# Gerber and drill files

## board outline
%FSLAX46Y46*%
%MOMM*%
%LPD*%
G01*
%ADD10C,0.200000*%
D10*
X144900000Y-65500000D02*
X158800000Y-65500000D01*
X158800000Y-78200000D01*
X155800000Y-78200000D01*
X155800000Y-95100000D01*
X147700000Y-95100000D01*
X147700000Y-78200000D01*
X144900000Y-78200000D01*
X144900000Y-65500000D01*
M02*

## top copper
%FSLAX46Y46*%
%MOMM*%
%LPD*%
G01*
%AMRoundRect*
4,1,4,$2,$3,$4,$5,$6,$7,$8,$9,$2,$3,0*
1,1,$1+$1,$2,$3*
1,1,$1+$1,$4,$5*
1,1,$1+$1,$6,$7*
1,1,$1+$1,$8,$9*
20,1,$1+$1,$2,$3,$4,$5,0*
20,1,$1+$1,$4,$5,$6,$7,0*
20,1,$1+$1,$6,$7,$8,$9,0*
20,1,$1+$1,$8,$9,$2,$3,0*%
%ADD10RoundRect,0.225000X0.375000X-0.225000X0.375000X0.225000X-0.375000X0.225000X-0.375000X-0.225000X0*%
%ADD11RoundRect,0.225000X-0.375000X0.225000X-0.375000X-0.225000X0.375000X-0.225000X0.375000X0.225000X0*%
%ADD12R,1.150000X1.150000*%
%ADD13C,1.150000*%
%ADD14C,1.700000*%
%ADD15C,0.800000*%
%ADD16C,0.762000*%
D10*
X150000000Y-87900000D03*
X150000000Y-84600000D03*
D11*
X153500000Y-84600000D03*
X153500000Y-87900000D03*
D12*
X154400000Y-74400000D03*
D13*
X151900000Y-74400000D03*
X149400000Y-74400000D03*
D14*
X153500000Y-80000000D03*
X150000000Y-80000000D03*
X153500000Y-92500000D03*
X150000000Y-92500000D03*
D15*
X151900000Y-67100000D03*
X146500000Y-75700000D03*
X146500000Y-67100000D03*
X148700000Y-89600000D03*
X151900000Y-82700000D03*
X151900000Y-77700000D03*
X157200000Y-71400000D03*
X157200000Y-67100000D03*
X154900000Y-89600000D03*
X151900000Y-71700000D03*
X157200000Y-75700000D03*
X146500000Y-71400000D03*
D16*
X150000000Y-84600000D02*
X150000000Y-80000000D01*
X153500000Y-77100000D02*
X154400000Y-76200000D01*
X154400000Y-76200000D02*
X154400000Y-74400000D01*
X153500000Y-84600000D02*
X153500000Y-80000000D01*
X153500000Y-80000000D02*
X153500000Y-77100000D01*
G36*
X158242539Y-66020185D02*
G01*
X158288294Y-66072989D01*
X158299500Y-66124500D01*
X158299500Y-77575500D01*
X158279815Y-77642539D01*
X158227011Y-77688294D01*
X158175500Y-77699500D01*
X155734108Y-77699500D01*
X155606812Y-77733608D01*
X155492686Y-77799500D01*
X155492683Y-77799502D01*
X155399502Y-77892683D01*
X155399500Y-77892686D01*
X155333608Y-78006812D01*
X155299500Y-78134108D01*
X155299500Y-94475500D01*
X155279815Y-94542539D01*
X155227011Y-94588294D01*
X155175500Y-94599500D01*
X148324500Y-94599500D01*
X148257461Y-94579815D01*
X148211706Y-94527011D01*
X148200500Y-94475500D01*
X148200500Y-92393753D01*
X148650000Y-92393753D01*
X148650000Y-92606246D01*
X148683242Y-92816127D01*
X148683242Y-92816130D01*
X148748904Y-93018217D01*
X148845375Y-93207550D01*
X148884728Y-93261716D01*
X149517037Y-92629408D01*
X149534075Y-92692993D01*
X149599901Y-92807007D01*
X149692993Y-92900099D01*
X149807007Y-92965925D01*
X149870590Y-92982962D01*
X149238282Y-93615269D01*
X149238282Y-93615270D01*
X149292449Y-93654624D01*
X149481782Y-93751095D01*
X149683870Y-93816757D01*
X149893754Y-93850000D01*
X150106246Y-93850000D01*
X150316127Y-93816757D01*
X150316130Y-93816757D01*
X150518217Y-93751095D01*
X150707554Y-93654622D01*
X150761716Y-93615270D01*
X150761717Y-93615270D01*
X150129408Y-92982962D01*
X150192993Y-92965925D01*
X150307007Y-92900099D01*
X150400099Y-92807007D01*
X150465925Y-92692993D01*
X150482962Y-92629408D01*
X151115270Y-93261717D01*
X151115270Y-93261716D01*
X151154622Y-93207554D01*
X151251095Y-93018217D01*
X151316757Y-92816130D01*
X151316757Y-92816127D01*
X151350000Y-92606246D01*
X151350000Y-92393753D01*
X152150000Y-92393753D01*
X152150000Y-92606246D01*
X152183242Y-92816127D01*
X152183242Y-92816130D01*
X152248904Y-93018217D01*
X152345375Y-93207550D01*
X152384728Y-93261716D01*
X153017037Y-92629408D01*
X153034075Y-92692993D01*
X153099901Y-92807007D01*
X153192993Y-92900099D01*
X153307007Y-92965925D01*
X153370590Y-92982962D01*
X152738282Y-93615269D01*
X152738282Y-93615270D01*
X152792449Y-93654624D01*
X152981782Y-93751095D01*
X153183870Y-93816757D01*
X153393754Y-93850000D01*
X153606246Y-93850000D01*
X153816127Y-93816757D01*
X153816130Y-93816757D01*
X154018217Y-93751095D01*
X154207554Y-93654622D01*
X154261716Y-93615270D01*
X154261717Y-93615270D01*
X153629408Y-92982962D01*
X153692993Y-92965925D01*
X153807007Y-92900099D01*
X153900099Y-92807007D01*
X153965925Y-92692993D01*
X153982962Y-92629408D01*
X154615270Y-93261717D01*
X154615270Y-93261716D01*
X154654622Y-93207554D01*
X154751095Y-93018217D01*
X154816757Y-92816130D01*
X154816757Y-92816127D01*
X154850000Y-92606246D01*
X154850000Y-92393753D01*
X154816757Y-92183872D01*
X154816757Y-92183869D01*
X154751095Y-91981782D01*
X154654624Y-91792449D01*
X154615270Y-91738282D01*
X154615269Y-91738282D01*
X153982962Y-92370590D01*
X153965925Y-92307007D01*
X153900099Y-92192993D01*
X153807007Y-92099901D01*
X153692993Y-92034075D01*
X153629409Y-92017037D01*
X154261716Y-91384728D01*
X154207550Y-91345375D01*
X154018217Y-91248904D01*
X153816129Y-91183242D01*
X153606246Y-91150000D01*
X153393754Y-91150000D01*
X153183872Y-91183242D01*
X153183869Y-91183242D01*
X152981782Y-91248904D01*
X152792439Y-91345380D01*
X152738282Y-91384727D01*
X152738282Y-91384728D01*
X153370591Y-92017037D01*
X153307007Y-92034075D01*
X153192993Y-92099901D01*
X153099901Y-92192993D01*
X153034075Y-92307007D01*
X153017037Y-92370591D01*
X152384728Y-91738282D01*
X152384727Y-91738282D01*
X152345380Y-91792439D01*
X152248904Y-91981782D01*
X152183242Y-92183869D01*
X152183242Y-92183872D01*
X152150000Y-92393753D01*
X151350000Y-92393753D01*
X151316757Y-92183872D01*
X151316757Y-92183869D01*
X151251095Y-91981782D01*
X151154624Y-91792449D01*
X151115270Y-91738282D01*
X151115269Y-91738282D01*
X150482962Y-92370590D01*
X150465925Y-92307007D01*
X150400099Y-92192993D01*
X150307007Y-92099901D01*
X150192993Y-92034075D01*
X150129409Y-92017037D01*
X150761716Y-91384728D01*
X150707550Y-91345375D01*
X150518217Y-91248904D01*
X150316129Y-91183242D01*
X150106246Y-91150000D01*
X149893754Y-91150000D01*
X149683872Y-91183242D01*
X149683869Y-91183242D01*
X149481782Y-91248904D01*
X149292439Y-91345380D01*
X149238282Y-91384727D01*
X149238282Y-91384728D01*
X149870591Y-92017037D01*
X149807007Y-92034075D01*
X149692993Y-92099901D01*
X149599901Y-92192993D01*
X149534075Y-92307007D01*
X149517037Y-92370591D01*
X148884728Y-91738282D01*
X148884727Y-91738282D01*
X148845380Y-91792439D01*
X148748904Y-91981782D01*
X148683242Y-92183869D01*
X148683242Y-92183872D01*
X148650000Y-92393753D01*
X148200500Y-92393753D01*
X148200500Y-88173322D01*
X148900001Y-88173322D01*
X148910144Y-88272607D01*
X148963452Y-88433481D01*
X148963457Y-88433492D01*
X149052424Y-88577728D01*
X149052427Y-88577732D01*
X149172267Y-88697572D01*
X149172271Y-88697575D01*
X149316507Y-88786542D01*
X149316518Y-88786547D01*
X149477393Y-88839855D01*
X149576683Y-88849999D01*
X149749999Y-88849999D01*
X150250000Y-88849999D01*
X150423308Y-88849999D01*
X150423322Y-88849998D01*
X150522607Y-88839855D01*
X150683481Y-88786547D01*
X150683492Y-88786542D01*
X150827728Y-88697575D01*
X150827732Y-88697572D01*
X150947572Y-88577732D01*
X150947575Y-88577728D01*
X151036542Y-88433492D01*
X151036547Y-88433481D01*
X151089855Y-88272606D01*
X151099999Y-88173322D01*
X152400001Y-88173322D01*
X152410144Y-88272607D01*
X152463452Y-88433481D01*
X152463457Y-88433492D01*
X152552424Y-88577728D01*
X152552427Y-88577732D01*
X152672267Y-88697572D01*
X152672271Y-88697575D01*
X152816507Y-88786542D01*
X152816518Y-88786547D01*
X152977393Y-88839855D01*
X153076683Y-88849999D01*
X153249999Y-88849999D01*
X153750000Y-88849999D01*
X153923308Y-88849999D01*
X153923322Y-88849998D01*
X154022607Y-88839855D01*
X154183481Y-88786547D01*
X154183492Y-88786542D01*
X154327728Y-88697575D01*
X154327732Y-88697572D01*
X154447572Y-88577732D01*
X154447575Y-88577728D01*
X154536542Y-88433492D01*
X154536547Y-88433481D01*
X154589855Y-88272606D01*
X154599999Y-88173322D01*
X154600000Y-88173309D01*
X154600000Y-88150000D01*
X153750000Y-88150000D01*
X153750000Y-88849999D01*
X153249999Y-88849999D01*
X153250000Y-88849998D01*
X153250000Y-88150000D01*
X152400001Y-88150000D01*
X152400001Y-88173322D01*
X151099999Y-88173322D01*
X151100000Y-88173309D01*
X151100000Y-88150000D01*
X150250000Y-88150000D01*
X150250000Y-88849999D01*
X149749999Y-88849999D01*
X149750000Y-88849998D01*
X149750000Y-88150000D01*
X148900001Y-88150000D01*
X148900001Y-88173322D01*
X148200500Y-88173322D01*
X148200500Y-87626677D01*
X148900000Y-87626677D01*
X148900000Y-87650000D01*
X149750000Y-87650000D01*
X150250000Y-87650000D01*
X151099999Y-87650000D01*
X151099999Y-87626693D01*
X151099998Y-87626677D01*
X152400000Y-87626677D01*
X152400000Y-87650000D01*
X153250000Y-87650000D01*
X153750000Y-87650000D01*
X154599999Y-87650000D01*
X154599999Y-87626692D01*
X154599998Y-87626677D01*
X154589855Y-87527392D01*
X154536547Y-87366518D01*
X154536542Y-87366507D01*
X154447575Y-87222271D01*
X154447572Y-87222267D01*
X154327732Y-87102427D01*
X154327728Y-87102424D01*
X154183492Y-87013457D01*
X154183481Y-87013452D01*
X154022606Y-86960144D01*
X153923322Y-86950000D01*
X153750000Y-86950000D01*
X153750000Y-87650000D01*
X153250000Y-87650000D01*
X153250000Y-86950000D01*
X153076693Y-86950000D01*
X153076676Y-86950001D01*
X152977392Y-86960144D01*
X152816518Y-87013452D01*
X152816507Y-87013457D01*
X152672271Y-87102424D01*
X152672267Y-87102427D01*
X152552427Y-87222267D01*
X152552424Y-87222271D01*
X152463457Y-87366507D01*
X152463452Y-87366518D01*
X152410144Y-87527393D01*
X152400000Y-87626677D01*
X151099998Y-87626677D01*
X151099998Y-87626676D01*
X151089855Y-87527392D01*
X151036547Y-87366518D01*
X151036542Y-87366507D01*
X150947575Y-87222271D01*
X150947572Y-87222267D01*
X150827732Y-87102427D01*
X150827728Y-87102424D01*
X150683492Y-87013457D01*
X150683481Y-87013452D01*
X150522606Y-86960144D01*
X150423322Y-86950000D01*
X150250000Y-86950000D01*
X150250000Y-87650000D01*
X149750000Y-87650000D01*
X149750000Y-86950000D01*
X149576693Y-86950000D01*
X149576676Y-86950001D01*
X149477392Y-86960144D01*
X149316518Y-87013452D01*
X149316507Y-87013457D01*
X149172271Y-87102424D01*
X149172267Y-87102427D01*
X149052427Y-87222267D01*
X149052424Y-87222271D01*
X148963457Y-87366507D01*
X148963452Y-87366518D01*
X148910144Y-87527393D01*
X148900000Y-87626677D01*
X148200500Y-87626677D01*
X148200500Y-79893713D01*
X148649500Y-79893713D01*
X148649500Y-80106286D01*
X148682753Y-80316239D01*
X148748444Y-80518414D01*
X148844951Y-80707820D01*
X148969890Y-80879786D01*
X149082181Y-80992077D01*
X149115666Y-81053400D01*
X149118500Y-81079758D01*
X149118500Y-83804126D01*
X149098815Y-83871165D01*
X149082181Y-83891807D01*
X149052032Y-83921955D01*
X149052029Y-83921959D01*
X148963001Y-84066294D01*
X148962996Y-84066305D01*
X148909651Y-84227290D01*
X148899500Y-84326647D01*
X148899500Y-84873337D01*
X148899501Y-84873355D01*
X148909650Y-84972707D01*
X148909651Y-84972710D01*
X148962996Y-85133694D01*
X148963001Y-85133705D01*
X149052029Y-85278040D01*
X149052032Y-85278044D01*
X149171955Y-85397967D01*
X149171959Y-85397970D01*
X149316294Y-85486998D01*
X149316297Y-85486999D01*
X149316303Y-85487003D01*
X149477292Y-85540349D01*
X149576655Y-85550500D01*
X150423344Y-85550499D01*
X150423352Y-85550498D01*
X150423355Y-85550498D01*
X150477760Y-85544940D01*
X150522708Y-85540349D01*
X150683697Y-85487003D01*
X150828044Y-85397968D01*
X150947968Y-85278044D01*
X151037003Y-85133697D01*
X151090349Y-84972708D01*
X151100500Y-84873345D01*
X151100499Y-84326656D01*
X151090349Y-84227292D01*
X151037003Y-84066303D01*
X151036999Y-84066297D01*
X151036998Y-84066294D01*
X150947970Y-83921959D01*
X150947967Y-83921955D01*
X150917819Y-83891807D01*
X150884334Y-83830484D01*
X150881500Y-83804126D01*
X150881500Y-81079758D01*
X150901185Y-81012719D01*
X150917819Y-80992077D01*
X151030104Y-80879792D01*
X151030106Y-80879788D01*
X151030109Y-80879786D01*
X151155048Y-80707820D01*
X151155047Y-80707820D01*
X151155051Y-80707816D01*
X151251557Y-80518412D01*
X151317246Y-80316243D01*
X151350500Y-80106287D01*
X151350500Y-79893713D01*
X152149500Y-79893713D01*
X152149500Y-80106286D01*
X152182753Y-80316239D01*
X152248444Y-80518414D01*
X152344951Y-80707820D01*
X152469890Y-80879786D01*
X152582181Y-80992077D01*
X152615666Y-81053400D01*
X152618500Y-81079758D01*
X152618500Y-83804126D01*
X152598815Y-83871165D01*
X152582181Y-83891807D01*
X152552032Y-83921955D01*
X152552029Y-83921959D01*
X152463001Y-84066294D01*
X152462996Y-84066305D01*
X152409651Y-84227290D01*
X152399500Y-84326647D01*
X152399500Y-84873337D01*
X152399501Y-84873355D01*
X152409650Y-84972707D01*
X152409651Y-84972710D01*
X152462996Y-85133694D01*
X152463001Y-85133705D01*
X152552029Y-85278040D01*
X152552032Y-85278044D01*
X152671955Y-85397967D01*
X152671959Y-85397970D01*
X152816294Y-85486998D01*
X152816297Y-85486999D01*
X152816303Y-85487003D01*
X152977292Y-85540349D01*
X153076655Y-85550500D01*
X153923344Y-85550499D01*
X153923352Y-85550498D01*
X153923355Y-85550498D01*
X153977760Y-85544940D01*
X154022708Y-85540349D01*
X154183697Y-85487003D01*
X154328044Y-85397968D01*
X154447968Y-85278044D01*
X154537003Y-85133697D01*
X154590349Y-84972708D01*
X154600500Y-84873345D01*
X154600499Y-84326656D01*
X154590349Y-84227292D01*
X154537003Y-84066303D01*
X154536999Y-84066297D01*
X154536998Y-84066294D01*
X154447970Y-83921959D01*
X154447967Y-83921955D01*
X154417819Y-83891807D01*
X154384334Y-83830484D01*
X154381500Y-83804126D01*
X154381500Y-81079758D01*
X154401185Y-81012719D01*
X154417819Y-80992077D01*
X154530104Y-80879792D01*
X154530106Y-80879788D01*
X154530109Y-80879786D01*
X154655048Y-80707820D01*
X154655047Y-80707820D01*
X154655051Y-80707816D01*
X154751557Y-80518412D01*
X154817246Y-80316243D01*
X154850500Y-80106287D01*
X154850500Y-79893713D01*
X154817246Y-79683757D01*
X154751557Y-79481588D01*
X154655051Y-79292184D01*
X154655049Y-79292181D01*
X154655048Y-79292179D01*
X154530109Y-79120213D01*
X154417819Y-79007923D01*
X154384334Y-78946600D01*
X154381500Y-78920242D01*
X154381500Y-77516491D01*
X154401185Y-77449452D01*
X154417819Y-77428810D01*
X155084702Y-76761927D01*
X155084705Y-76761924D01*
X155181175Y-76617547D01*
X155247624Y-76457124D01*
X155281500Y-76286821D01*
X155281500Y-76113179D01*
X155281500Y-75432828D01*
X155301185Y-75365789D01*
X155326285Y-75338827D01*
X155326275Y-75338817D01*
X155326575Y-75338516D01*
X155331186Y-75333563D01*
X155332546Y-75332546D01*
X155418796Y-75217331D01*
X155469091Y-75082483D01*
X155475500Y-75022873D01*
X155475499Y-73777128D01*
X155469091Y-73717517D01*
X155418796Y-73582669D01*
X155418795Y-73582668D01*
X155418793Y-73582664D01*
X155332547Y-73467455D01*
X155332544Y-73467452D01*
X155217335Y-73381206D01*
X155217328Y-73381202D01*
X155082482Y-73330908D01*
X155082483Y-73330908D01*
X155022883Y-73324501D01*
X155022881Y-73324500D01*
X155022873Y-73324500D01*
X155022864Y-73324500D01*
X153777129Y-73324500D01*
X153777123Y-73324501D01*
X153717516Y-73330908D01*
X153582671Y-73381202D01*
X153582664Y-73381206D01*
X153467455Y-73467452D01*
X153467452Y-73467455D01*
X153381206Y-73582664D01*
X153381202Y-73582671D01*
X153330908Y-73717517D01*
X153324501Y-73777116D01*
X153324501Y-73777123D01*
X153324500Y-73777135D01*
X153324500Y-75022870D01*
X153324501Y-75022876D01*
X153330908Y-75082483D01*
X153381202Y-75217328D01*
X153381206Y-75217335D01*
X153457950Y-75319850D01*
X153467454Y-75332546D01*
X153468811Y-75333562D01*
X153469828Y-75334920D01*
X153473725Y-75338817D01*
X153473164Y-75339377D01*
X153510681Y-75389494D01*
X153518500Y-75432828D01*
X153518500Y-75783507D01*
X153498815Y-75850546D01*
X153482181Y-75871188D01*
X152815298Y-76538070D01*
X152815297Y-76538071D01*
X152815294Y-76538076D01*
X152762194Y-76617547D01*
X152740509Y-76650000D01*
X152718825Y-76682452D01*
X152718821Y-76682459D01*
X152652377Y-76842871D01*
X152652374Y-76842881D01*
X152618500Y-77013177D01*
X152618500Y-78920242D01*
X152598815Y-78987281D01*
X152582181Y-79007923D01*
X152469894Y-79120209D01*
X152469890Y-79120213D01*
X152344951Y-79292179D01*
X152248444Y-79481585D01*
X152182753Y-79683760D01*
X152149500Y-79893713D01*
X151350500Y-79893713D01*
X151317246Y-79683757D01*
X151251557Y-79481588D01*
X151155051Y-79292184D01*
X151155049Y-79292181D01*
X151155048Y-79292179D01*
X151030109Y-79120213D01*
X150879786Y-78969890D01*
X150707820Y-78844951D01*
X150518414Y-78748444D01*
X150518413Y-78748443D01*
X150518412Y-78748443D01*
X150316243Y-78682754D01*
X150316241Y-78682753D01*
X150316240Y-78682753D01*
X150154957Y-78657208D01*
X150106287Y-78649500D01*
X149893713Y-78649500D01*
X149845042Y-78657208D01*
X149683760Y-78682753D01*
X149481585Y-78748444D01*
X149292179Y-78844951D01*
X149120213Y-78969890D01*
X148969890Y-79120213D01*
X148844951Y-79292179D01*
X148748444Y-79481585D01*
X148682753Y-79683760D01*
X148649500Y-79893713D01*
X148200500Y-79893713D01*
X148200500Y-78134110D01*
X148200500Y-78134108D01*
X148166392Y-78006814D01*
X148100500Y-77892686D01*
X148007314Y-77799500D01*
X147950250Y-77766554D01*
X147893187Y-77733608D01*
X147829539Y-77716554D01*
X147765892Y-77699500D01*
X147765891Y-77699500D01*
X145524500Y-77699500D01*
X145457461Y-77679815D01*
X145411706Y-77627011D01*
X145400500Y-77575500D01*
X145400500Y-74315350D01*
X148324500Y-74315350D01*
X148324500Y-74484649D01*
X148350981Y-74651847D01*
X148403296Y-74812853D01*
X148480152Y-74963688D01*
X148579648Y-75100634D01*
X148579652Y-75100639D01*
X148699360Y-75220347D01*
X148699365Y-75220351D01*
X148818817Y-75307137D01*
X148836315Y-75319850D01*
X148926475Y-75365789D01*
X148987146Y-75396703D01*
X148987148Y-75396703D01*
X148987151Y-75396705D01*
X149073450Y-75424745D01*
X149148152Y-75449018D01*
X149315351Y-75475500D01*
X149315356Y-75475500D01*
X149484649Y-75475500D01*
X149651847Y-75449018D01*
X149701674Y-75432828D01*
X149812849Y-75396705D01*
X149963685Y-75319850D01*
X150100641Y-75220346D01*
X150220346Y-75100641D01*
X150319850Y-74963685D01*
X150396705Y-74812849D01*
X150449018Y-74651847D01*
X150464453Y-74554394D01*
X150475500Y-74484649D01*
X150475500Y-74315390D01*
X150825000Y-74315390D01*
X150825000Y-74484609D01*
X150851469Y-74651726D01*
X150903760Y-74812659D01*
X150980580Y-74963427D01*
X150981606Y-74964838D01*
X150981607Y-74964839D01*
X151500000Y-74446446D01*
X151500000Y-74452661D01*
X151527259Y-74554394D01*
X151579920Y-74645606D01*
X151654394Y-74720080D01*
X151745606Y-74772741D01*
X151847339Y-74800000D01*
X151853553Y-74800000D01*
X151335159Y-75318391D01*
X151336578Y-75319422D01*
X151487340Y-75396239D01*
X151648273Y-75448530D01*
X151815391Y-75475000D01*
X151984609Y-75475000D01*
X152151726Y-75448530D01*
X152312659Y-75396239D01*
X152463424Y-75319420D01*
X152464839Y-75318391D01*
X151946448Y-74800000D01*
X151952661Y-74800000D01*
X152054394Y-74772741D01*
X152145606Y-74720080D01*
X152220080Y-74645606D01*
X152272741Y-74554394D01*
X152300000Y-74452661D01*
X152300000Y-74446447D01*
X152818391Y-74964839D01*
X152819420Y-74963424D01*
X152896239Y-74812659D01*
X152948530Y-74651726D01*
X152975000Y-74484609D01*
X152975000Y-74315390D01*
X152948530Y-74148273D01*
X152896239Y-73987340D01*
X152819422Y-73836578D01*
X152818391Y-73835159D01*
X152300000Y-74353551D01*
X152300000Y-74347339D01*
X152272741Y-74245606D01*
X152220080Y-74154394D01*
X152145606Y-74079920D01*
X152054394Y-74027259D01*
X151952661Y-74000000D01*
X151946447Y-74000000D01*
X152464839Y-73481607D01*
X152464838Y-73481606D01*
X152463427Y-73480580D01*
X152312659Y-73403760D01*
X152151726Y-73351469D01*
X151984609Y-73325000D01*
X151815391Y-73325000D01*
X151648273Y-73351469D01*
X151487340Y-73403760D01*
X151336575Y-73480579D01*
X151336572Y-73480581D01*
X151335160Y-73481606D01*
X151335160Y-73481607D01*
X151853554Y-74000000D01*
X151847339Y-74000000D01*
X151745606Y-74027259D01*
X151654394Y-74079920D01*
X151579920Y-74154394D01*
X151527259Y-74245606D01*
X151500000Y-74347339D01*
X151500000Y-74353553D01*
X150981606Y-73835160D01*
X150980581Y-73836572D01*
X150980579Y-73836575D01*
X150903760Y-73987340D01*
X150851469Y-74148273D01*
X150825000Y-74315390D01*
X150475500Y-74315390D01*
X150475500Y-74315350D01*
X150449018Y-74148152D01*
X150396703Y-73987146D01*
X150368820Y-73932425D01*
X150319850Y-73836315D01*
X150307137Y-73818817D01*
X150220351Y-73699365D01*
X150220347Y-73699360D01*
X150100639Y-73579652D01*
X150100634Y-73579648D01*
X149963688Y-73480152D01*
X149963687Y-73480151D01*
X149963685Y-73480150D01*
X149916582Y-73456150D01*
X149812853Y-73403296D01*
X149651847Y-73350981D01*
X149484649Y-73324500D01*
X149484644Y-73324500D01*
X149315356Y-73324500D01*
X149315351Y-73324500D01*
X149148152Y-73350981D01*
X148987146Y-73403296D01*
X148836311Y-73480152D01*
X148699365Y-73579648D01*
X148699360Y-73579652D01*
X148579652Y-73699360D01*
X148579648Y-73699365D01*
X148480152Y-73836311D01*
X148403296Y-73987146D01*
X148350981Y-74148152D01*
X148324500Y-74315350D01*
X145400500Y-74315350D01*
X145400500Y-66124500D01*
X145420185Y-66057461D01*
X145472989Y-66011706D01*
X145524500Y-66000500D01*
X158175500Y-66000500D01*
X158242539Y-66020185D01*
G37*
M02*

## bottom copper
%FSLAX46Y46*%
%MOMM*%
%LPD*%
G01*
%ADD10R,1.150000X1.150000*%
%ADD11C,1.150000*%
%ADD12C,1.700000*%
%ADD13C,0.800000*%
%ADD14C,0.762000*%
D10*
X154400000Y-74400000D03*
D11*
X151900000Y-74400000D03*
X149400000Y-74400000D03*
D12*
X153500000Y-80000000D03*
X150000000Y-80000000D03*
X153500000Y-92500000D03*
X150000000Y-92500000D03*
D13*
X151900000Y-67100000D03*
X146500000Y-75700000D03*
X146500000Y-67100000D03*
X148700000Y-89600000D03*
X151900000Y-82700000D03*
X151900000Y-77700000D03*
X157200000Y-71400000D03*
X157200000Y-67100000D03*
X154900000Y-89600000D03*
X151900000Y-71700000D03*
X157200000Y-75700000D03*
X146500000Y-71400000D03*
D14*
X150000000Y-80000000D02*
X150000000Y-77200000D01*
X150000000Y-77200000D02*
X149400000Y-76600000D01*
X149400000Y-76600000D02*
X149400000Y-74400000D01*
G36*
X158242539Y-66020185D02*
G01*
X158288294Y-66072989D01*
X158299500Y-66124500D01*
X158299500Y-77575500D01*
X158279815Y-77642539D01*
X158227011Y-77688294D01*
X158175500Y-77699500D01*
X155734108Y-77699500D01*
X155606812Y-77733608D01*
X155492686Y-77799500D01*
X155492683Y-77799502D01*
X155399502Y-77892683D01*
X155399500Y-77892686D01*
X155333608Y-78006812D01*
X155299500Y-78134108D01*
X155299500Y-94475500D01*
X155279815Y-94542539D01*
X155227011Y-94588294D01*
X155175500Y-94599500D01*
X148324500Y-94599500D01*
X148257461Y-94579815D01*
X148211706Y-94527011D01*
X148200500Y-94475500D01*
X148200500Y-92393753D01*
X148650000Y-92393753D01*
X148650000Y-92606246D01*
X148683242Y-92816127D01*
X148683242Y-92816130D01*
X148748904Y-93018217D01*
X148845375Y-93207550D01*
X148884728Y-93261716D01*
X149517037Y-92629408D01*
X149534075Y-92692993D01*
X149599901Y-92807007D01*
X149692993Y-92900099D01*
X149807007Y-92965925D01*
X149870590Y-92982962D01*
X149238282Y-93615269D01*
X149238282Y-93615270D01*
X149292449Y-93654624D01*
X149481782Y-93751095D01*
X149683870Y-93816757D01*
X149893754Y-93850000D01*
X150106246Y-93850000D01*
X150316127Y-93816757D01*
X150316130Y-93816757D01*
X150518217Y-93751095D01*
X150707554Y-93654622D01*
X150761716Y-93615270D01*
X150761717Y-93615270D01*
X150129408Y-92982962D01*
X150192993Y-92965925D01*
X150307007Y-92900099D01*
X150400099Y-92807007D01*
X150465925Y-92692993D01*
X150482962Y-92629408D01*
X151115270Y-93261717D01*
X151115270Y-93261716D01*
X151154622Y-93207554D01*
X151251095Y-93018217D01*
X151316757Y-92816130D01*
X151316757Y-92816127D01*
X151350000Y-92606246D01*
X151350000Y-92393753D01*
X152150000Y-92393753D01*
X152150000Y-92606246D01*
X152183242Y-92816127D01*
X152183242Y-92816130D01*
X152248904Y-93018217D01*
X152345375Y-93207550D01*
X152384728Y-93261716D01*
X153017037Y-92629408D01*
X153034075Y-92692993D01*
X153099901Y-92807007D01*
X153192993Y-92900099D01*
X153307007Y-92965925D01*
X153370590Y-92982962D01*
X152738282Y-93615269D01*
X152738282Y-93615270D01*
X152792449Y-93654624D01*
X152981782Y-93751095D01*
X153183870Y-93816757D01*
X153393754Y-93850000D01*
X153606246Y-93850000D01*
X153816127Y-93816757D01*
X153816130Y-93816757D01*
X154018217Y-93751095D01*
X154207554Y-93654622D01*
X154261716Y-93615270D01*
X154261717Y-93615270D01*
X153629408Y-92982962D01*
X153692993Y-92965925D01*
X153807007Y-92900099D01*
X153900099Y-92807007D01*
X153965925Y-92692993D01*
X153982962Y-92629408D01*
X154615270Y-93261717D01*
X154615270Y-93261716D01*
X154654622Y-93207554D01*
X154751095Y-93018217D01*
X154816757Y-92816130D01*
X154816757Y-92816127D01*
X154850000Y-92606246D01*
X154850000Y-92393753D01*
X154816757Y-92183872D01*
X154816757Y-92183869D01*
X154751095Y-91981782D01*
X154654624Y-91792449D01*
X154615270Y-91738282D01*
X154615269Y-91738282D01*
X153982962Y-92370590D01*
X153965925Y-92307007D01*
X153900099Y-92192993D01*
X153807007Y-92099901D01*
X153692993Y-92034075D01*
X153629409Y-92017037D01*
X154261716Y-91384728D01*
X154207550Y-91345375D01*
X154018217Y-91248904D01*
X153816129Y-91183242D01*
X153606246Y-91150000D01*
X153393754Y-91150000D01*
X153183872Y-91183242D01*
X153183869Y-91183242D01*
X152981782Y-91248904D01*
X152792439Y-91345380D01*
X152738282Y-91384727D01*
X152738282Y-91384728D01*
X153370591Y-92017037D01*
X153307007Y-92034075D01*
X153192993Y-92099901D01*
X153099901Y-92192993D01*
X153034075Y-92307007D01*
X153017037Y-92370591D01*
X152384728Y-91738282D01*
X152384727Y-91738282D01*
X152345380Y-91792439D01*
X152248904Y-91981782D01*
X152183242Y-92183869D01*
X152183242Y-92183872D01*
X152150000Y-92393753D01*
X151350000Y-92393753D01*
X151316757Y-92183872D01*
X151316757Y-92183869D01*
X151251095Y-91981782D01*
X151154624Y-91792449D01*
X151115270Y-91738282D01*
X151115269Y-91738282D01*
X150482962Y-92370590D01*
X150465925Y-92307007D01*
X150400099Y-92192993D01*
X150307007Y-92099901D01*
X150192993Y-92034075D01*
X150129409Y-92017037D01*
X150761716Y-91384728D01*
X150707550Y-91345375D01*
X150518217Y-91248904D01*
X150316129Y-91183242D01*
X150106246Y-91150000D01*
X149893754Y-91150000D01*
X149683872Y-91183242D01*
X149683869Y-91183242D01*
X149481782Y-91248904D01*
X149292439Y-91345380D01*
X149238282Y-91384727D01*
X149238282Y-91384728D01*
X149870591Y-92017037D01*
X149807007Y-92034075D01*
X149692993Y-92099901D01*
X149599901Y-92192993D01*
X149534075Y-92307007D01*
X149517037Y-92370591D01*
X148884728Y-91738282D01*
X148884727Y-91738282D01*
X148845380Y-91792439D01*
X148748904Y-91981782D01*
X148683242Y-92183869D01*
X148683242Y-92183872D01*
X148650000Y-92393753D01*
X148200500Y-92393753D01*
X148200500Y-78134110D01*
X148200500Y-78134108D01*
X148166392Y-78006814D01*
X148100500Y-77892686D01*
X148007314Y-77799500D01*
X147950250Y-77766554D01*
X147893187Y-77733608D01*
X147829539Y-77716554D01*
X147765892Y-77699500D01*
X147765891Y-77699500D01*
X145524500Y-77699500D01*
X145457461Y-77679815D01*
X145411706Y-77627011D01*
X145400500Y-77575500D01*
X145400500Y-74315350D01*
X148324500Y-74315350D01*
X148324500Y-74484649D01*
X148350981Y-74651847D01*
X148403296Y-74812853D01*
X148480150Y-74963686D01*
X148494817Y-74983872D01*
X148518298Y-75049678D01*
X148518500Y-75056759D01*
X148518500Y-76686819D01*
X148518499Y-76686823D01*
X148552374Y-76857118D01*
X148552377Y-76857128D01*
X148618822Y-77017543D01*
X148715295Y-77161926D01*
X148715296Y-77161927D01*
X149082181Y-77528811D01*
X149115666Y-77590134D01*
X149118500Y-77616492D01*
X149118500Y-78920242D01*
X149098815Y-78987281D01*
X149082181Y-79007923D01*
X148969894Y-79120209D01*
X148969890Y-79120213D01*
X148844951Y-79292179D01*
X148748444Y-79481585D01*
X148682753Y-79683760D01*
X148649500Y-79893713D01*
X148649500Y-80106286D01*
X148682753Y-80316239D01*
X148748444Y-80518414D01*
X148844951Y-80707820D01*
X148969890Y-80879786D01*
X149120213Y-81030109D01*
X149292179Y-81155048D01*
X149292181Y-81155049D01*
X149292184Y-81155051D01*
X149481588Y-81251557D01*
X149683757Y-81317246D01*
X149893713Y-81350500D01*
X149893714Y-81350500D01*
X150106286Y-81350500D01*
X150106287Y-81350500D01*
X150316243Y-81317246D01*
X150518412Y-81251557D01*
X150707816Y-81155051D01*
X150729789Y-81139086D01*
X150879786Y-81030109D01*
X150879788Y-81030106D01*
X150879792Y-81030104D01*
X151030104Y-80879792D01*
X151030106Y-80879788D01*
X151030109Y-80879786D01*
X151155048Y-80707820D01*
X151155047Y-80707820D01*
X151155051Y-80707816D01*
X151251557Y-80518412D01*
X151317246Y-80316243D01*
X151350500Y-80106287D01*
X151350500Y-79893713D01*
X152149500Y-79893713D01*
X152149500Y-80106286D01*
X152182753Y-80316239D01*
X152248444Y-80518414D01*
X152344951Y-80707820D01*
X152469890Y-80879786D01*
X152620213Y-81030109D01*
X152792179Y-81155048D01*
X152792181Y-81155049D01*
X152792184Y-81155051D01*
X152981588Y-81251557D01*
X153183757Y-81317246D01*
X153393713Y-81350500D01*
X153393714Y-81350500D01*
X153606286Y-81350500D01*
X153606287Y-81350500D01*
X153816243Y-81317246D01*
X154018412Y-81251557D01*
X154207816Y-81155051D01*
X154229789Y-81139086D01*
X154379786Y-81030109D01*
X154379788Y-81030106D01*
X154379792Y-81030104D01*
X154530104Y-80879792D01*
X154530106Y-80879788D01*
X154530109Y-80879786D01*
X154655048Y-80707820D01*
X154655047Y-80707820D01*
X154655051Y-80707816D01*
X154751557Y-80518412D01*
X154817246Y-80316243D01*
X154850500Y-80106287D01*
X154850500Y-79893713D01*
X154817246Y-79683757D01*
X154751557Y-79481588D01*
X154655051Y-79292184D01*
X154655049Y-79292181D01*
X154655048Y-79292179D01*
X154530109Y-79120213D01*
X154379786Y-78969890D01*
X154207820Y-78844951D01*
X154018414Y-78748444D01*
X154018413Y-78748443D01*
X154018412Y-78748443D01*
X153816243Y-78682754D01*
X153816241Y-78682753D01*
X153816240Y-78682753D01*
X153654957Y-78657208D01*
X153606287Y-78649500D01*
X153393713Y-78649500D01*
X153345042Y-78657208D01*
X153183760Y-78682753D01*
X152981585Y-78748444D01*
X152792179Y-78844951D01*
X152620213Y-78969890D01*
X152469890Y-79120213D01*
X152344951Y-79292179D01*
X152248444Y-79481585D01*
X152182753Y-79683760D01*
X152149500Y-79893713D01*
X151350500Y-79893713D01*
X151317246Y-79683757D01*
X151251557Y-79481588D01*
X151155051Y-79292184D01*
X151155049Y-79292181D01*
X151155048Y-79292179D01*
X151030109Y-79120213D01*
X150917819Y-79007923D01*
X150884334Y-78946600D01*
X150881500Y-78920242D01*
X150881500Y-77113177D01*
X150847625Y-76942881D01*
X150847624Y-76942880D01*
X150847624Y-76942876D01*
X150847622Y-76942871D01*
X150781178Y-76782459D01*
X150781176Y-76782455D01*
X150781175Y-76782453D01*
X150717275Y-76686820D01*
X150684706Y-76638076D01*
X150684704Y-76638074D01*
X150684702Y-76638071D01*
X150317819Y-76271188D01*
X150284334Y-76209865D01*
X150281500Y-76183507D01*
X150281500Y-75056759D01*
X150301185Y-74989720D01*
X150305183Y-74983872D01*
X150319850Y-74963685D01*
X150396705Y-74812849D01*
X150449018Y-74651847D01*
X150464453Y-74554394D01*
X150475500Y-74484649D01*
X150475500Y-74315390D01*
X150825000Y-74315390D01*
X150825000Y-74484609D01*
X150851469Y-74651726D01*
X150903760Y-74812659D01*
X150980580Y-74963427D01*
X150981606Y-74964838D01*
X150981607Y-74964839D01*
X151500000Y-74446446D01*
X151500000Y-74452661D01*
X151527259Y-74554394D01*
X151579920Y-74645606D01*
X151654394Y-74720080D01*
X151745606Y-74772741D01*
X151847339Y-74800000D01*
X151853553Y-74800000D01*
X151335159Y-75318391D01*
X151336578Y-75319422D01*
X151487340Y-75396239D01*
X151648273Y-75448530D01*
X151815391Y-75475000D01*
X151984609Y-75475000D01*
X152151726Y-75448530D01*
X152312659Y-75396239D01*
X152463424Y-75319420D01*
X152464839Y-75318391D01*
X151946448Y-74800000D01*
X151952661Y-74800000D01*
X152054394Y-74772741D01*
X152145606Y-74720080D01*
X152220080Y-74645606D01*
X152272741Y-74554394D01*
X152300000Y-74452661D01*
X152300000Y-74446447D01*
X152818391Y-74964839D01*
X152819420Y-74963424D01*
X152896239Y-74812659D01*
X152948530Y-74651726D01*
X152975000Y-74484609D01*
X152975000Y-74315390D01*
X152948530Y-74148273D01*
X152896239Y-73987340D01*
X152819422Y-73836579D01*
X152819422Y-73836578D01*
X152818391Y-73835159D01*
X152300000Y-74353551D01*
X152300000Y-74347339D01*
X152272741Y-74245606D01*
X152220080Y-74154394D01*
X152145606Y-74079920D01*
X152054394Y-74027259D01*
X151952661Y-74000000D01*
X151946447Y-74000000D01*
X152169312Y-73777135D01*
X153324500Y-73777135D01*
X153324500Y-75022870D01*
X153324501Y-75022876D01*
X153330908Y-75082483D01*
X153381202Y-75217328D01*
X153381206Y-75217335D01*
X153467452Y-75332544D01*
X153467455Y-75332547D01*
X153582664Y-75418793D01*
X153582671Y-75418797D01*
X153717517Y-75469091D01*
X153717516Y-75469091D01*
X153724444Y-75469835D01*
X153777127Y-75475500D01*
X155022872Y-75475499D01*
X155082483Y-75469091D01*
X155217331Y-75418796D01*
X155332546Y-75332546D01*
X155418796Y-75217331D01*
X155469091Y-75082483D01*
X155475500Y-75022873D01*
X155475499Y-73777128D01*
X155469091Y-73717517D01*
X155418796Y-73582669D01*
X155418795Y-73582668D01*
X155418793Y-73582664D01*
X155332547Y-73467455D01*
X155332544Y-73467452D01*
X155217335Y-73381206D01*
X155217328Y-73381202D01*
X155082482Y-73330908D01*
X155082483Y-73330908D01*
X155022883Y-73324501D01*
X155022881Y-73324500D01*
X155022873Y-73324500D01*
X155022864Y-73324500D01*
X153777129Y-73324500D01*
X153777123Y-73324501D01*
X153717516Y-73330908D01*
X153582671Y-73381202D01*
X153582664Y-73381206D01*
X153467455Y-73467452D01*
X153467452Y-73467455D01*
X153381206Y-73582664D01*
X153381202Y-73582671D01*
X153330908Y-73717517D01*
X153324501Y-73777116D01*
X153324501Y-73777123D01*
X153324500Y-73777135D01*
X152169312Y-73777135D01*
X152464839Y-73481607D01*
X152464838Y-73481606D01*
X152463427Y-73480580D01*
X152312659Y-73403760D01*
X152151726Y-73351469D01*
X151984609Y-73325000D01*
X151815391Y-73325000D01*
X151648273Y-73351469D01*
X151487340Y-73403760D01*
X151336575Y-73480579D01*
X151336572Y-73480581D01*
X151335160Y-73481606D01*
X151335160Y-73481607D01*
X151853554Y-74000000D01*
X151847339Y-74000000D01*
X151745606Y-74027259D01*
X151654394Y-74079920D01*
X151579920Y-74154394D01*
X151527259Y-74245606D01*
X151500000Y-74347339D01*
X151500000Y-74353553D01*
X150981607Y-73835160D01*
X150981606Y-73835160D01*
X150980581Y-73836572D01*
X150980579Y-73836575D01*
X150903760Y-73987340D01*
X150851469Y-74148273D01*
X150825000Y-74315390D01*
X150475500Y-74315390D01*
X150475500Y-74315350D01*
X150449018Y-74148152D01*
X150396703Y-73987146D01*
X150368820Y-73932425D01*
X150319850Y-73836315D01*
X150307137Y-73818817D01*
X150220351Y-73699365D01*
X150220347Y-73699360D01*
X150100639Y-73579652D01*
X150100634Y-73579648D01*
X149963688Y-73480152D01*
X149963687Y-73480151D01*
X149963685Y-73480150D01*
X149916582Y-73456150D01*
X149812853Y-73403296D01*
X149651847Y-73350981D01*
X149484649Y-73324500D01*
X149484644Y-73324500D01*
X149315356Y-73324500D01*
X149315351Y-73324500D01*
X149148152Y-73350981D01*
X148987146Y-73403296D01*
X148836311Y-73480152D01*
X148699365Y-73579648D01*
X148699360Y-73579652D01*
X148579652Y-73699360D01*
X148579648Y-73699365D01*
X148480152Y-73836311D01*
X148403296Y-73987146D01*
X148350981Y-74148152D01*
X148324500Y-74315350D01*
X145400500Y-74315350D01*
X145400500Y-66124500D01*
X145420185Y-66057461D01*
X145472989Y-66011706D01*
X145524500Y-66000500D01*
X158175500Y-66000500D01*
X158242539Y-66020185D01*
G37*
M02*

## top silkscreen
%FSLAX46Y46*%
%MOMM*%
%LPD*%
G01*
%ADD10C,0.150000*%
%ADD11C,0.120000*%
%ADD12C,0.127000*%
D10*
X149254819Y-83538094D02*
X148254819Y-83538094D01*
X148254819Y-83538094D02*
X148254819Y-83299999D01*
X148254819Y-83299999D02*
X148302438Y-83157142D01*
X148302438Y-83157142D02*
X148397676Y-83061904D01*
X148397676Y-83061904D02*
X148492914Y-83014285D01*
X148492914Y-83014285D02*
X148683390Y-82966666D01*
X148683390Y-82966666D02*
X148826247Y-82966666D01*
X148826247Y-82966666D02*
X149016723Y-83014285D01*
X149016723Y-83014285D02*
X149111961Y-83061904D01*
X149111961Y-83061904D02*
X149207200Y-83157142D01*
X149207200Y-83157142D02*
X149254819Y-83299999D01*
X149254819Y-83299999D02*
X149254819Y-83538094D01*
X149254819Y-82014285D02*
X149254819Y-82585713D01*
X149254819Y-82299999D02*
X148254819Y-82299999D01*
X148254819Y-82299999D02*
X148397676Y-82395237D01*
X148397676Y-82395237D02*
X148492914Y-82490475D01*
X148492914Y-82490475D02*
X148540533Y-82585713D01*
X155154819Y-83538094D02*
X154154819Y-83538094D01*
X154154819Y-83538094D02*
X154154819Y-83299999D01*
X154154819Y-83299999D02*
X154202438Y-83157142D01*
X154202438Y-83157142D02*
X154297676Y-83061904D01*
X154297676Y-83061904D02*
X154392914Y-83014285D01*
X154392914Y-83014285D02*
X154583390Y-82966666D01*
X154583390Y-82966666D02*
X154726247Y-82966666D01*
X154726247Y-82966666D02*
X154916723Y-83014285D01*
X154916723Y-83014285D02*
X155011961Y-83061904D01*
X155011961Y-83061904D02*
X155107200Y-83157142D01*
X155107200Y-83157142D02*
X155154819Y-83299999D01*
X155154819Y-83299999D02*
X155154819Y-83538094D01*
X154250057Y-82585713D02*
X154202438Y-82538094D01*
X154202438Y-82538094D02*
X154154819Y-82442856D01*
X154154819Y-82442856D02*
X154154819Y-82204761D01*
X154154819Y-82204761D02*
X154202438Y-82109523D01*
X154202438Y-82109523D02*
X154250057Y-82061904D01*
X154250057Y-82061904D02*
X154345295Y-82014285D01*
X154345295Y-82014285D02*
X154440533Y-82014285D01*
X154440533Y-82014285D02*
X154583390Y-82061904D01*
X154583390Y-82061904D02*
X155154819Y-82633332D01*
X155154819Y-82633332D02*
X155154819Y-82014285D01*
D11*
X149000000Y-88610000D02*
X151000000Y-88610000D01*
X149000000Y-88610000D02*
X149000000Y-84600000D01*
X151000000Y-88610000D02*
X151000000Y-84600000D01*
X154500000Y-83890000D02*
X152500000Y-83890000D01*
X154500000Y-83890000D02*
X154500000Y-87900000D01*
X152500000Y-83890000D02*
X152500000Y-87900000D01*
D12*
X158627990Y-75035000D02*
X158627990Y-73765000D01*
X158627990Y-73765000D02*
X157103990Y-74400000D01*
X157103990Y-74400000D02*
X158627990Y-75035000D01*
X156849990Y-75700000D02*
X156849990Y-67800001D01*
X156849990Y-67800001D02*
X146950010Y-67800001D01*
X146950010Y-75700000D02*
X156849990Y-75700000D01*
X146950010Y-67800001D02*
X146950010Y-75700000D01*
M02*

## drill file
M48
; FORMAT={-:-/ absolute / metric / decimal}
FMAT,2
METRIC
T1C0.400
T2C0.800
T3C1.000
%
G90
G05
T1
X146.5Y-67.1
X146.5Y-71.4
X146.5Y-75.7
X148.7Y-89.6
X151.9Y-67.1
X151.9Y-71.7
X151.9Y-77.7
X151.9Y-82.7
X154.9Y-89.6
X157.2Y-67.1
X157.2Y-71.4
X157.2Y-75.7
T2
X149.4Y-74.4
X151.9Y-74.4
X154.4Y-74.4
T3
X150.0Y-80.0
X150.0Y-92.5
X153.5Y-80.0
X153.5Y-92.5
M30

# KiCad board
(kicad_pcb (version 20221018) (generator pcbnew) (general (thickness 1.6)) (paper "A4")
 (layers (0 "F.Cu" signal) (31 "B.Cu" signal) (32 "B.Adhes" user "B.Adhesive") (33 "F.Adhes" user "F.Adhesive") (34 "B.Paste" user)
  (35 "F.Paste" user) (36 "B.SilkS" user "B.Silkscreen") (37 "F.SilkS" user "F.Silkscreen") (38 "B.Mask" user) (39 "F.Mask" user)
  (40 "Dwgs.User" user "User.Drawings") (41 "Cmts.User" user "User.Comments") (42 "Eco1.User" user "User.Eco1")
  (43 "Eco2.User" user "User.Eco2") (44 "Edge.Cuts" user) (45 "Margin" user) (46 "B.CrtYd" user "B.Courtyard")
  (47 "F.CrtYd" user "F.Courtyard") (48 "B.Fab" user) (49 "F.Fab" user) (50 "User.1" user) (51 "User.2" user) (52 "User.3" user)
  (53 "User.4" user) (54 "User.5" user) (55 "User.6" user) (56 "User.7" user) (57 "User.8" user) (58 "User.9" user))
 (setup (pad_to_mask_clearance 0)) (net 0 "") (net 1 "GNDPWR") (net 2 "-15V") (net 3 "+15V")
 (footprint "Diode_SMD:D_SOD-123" (layer "F.Cu") (at 150 86.25 90)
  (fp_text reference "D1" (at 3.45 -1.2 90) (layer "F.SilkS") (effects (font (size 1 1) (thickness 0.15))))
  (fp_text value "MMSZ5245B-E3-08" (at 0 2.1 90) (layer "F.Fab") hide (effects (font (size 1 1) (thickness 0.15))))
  (fp_line (start -2.36 -1) (end -2.36 1) (stroke (width 0.12) (type solid)) (layer "F.SilkS"))
  (fp_line (start -2.36 -1) (end 1.65 -1) (stroke (width 0.12) (type solid)) (layer "F.SilkS"))
  (fp_line (start -2.36 1) (end 1.65 1) (stroke (width 0.12) (type solid)) (layer "F.SilkS"))
  (pad "1" smd roundrect (at -1.65 0 90) (size 0.9 1.2) (layers "F.Cu" "F.Paste" "F.Mask") (roundrect_rratio 0.25) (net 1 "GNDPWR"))
  (pad "2" smd roundrect (at 1.65 0 90) (size 0.9 1.2) (layers "F.Cu" "F.Paste" "F.Mask") (roundrect_rratio 0.25) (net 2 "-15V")))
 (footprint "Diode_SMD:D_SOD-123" (layer "F.Cu") (at 153.5 86.25 -90)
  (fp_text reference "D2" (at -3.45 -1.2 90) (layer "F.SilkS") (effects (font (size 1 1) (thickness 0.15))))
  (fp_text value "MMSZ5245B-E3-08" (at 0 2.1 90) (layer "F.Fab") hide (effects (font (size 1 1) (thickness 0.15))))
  (fp_line (start -2.36 -1) (end -2.36 1) (stroke (width 0.12) (type solid)) (layer "F.SilkS"))
  (fp_line (start -2.36 -1) (end 1.65 -1) (stroke (width 0.12) (type solid)) (layer "F.SilkS"))
  (fp_line (start -2.36 1) (end 1.65 1) (stroke (width 0.12) (type solid)) (layer "F.SilkS"))
  (pad "1" smd roundrect (at -1.65 0 270) (size 0.9 1.2) (layers "F.Cu" "F.Paste" "F.Mask") (roundrect_rratio 0.25) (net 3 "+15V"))
  (pad "2" smd roundrect (at 1.65 0 270) (size 0.9 1.2) (layers "F.Cu" "F.Paste" "F.Mask") (roundrect_rratio 0.25) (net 1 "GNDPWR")))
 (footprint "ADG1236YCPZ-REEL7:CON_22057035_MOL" (layer "F.Cu") (at 154.4 74.4 180)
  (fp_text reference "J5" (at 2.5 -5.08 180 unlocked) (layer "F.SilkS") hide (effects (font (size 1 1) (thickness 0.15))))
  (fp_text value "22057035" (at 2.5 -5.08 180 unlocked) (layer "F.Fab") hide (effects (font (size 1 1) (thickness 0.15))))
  (fp_line (start -4.22799 -0.635) (end -4.22799 0.635) (stroke (width 0.127) (type solid)) (layer "F.SilkS"))
  (fp_line (start -4.22799 0.635) (end -2.70399 0) (stroke (width 0.127) (type solid)) (layer "F.SilkS"))
  (fp_line (start -2.70399 0) (end -4.22799 -0.635) (stroke (width 0.127) (type solid)) (layer "F.SilkS"))
  (fp_line (start -2.44999 -1.3) (end -2.44999 6.599999) (stroke (width 0.127) (type solid)) (layer "F.SilkS"))
  (fp_line (start -2.44999 6.599999) (end 7.44999 6.599999) (stroke (width 0.127) (type solid)) (layer "F.SilkS"))
  (fp_line (start 7.44999 -1.3) (end -2.44999 -1.3) (stroke (width 0.127) (type solid)) (layer "F.SilkS"))
  (fp_line (start 7.44999 6.599999) (end 7.44999 -1.3) (stroke (width 0.127) (type solid)) (layer "F.SilkS"))
  (pad "1" thru_hole rect (at 0 0 180) (size 1.15 1.15) (drill 0.8) (layers "*.Cu" "*.Mask") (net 3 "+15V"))
  (pad "2" thru_hole circle (at 2.5 0 180) (size 1.15 1.15) (drill 0.8) (layers "*.Cu" "*.Mask") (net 1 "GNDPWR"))
  (pad "3" thru_hole circle (at 5 0 180) (size 1.15 1.15) (drill 0.8) (layers "*.Cu" "*.Mask") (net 2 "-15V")))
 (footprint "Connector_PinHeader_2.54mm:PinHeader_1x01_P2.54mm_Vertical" (layer "B.Cu") (at 153.5 80 180)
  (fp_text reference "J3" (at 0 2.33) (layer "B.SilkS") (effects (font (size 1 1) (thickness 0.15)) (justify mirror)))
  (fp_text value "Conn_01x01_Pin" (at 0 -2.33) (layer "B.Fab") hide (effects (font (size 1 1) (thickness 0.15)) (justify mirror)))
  (pad "1" thru_hole circle (at 0 0 180) (size 1.7 1.7) (drill 1) (layers "*.Cu" "*.Mask") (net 3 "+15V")))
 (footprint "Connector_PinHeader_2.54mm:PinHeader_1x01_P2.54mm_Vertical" (layer "B.Cu") (at 150 80 180)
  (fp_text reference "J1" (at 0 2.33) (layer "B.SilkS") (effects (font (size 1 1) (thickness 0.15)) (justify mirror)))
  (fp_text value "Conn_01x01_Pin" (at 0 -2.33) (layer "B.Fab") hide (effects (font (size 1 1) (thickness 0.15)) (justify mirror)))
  (pad "1" thru_hole circle (at 0 0 180) (size 1.7 1.7) (drill 1) (layers "*.Cu" "*.Mask") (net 2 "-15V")))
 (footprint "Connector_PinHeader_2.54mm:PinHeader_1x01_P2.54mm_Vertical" (layer "B.Cu") (at 153.5 92.5 180)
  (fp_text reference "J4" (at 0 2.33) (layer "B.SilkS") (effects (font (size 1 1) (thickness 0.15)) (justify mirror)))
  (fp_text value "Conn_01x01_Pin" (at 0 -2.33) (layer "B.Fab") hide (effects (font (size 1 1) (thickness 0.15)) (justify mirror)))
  (pad "1" thru_hole circle (at 0 0 180) (size 1.7 1.7) (drill 1) (layers "*.Cu" "*.Mask") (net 1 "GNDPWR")))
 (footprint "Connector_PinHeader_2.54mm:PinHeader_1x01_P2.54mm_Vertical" (layer "B.Cu") (at 150 92.5 180)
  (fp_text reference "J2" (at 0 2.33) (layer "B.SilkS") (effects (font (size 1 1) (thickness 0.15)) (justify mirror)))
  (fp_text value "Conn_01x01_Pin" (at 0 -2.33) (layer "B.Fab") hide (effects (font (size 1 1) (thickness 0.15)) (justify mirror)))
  (pad "1" thru_hole circle (at 0 0 180) (size 1.7 1.7) (drill 1) (layers "*.Cu" "*.Mask") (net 1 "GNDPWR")))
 (gr_poly
  (pts (xy 144.9 65.5) (xy 158.8 65.5) (xy 158.8 78.2) (xy 155.8 78.2) (xy 155.8 95.1) (xy 147.7 95.1) (xy 147.7 78.2) (xy 144.9 78.2))
  (stroke (width 0.2) (type solid)) (fill none) (layer "Edge.Cuts"))
 (via (at 151.9 67.1) (size 0.8) (drill 0.4) (layers "F.Cu" "B.Cu") (free) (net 1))
 (via (at 146.5 75.7) (size 0.8) (drill 0.4) (layers "F.Cu" "B.Cu") (free) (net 1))
 (via (at 146.5 67.1) (size 0.8) (drill 0.4) (layers "F.Cu" "B.Cu") (free) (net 1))
 (via (at 148.7 89.6) (size 0.8) (drill 0.4) (layers "F.Cu" "B.Cu") (free) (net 1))
 (via (at 151.9 82.7) (size 0.8) (drill 0.4) (layers "F.Cu" "B.Cu") (free) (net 1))
 (via (at 151.9 77.7) (size 0.8) (drill 0.4) (layers "F.Cu" "B.Cu") (free) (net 1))
 (via (at 157.2 71.4) (size 0.8) (drill 0.4) (layers "F.Cu" "B.Cu") (free) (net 1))
 (via (at 157.2 67.1) (size 0.8) (drill 0.4) (layers "F.Cu" "B.Cu") (free) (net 1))
 (via (at 154.9 89.6) (size 0.8) (drill 0.4) (layers "F.Cu" "B.Cu") (free) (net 1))
 (via (at 151.9 71.7) (size 0.8) (drill 0.4) (layers "F.Cu" "B.Cu") (free) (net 1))
 (via (at 157.2 75.7) (size 0.8) (drill 0.4) (layers "F.Cu" "B.Cu") (free) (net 1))
 (via (at 146.5 71.4) (size 0.8) (drill 0.4) (layers "F.Cu" "B.Cu") (free) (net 1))
 (segment (start 150 84.6) (end 150 80) (width 0.762) (layer "F.Cu") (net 2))
 (segment (start 150 80) (end 150 77.2) (width 0.762) (layer "B.Cu") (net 2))
 (segment (start 150 77.2) (end 149.4 76.6) (width 0.762) (layer "B.Cu") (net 2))
 (segment (start 149.4 76.6) (end 149.4 74.4) (width 0.762) (layer "B.Cu") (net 2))
 (segment (start 153.5 77.1) (end 154.4 76.2) (width 0.762) (layer "F.Cu") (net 3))
 (segment (start 154.4 76.2) (end 154.4 74.4) (width 0.762) (layer "F.Cu") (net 3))
 (segment (start 153.5 84.6) (end 153.5 80) (width 0.762) (layer "F.Cu") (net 3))
 (segment (start 153.5 80) (end 153.5 77.1) (width 0.762) (layer "F.Cu") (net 3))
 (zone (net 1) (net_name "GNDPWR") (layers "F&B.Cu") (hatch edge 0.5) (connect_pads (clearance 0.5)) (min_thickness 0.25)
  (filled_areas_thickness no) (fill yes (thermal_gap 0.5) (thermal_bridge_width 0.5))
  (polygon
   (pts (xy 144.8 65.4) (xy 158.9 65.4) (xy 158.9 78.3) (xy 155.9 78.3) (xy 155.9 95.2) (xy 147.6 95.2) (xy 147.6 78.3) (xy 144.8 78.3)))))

